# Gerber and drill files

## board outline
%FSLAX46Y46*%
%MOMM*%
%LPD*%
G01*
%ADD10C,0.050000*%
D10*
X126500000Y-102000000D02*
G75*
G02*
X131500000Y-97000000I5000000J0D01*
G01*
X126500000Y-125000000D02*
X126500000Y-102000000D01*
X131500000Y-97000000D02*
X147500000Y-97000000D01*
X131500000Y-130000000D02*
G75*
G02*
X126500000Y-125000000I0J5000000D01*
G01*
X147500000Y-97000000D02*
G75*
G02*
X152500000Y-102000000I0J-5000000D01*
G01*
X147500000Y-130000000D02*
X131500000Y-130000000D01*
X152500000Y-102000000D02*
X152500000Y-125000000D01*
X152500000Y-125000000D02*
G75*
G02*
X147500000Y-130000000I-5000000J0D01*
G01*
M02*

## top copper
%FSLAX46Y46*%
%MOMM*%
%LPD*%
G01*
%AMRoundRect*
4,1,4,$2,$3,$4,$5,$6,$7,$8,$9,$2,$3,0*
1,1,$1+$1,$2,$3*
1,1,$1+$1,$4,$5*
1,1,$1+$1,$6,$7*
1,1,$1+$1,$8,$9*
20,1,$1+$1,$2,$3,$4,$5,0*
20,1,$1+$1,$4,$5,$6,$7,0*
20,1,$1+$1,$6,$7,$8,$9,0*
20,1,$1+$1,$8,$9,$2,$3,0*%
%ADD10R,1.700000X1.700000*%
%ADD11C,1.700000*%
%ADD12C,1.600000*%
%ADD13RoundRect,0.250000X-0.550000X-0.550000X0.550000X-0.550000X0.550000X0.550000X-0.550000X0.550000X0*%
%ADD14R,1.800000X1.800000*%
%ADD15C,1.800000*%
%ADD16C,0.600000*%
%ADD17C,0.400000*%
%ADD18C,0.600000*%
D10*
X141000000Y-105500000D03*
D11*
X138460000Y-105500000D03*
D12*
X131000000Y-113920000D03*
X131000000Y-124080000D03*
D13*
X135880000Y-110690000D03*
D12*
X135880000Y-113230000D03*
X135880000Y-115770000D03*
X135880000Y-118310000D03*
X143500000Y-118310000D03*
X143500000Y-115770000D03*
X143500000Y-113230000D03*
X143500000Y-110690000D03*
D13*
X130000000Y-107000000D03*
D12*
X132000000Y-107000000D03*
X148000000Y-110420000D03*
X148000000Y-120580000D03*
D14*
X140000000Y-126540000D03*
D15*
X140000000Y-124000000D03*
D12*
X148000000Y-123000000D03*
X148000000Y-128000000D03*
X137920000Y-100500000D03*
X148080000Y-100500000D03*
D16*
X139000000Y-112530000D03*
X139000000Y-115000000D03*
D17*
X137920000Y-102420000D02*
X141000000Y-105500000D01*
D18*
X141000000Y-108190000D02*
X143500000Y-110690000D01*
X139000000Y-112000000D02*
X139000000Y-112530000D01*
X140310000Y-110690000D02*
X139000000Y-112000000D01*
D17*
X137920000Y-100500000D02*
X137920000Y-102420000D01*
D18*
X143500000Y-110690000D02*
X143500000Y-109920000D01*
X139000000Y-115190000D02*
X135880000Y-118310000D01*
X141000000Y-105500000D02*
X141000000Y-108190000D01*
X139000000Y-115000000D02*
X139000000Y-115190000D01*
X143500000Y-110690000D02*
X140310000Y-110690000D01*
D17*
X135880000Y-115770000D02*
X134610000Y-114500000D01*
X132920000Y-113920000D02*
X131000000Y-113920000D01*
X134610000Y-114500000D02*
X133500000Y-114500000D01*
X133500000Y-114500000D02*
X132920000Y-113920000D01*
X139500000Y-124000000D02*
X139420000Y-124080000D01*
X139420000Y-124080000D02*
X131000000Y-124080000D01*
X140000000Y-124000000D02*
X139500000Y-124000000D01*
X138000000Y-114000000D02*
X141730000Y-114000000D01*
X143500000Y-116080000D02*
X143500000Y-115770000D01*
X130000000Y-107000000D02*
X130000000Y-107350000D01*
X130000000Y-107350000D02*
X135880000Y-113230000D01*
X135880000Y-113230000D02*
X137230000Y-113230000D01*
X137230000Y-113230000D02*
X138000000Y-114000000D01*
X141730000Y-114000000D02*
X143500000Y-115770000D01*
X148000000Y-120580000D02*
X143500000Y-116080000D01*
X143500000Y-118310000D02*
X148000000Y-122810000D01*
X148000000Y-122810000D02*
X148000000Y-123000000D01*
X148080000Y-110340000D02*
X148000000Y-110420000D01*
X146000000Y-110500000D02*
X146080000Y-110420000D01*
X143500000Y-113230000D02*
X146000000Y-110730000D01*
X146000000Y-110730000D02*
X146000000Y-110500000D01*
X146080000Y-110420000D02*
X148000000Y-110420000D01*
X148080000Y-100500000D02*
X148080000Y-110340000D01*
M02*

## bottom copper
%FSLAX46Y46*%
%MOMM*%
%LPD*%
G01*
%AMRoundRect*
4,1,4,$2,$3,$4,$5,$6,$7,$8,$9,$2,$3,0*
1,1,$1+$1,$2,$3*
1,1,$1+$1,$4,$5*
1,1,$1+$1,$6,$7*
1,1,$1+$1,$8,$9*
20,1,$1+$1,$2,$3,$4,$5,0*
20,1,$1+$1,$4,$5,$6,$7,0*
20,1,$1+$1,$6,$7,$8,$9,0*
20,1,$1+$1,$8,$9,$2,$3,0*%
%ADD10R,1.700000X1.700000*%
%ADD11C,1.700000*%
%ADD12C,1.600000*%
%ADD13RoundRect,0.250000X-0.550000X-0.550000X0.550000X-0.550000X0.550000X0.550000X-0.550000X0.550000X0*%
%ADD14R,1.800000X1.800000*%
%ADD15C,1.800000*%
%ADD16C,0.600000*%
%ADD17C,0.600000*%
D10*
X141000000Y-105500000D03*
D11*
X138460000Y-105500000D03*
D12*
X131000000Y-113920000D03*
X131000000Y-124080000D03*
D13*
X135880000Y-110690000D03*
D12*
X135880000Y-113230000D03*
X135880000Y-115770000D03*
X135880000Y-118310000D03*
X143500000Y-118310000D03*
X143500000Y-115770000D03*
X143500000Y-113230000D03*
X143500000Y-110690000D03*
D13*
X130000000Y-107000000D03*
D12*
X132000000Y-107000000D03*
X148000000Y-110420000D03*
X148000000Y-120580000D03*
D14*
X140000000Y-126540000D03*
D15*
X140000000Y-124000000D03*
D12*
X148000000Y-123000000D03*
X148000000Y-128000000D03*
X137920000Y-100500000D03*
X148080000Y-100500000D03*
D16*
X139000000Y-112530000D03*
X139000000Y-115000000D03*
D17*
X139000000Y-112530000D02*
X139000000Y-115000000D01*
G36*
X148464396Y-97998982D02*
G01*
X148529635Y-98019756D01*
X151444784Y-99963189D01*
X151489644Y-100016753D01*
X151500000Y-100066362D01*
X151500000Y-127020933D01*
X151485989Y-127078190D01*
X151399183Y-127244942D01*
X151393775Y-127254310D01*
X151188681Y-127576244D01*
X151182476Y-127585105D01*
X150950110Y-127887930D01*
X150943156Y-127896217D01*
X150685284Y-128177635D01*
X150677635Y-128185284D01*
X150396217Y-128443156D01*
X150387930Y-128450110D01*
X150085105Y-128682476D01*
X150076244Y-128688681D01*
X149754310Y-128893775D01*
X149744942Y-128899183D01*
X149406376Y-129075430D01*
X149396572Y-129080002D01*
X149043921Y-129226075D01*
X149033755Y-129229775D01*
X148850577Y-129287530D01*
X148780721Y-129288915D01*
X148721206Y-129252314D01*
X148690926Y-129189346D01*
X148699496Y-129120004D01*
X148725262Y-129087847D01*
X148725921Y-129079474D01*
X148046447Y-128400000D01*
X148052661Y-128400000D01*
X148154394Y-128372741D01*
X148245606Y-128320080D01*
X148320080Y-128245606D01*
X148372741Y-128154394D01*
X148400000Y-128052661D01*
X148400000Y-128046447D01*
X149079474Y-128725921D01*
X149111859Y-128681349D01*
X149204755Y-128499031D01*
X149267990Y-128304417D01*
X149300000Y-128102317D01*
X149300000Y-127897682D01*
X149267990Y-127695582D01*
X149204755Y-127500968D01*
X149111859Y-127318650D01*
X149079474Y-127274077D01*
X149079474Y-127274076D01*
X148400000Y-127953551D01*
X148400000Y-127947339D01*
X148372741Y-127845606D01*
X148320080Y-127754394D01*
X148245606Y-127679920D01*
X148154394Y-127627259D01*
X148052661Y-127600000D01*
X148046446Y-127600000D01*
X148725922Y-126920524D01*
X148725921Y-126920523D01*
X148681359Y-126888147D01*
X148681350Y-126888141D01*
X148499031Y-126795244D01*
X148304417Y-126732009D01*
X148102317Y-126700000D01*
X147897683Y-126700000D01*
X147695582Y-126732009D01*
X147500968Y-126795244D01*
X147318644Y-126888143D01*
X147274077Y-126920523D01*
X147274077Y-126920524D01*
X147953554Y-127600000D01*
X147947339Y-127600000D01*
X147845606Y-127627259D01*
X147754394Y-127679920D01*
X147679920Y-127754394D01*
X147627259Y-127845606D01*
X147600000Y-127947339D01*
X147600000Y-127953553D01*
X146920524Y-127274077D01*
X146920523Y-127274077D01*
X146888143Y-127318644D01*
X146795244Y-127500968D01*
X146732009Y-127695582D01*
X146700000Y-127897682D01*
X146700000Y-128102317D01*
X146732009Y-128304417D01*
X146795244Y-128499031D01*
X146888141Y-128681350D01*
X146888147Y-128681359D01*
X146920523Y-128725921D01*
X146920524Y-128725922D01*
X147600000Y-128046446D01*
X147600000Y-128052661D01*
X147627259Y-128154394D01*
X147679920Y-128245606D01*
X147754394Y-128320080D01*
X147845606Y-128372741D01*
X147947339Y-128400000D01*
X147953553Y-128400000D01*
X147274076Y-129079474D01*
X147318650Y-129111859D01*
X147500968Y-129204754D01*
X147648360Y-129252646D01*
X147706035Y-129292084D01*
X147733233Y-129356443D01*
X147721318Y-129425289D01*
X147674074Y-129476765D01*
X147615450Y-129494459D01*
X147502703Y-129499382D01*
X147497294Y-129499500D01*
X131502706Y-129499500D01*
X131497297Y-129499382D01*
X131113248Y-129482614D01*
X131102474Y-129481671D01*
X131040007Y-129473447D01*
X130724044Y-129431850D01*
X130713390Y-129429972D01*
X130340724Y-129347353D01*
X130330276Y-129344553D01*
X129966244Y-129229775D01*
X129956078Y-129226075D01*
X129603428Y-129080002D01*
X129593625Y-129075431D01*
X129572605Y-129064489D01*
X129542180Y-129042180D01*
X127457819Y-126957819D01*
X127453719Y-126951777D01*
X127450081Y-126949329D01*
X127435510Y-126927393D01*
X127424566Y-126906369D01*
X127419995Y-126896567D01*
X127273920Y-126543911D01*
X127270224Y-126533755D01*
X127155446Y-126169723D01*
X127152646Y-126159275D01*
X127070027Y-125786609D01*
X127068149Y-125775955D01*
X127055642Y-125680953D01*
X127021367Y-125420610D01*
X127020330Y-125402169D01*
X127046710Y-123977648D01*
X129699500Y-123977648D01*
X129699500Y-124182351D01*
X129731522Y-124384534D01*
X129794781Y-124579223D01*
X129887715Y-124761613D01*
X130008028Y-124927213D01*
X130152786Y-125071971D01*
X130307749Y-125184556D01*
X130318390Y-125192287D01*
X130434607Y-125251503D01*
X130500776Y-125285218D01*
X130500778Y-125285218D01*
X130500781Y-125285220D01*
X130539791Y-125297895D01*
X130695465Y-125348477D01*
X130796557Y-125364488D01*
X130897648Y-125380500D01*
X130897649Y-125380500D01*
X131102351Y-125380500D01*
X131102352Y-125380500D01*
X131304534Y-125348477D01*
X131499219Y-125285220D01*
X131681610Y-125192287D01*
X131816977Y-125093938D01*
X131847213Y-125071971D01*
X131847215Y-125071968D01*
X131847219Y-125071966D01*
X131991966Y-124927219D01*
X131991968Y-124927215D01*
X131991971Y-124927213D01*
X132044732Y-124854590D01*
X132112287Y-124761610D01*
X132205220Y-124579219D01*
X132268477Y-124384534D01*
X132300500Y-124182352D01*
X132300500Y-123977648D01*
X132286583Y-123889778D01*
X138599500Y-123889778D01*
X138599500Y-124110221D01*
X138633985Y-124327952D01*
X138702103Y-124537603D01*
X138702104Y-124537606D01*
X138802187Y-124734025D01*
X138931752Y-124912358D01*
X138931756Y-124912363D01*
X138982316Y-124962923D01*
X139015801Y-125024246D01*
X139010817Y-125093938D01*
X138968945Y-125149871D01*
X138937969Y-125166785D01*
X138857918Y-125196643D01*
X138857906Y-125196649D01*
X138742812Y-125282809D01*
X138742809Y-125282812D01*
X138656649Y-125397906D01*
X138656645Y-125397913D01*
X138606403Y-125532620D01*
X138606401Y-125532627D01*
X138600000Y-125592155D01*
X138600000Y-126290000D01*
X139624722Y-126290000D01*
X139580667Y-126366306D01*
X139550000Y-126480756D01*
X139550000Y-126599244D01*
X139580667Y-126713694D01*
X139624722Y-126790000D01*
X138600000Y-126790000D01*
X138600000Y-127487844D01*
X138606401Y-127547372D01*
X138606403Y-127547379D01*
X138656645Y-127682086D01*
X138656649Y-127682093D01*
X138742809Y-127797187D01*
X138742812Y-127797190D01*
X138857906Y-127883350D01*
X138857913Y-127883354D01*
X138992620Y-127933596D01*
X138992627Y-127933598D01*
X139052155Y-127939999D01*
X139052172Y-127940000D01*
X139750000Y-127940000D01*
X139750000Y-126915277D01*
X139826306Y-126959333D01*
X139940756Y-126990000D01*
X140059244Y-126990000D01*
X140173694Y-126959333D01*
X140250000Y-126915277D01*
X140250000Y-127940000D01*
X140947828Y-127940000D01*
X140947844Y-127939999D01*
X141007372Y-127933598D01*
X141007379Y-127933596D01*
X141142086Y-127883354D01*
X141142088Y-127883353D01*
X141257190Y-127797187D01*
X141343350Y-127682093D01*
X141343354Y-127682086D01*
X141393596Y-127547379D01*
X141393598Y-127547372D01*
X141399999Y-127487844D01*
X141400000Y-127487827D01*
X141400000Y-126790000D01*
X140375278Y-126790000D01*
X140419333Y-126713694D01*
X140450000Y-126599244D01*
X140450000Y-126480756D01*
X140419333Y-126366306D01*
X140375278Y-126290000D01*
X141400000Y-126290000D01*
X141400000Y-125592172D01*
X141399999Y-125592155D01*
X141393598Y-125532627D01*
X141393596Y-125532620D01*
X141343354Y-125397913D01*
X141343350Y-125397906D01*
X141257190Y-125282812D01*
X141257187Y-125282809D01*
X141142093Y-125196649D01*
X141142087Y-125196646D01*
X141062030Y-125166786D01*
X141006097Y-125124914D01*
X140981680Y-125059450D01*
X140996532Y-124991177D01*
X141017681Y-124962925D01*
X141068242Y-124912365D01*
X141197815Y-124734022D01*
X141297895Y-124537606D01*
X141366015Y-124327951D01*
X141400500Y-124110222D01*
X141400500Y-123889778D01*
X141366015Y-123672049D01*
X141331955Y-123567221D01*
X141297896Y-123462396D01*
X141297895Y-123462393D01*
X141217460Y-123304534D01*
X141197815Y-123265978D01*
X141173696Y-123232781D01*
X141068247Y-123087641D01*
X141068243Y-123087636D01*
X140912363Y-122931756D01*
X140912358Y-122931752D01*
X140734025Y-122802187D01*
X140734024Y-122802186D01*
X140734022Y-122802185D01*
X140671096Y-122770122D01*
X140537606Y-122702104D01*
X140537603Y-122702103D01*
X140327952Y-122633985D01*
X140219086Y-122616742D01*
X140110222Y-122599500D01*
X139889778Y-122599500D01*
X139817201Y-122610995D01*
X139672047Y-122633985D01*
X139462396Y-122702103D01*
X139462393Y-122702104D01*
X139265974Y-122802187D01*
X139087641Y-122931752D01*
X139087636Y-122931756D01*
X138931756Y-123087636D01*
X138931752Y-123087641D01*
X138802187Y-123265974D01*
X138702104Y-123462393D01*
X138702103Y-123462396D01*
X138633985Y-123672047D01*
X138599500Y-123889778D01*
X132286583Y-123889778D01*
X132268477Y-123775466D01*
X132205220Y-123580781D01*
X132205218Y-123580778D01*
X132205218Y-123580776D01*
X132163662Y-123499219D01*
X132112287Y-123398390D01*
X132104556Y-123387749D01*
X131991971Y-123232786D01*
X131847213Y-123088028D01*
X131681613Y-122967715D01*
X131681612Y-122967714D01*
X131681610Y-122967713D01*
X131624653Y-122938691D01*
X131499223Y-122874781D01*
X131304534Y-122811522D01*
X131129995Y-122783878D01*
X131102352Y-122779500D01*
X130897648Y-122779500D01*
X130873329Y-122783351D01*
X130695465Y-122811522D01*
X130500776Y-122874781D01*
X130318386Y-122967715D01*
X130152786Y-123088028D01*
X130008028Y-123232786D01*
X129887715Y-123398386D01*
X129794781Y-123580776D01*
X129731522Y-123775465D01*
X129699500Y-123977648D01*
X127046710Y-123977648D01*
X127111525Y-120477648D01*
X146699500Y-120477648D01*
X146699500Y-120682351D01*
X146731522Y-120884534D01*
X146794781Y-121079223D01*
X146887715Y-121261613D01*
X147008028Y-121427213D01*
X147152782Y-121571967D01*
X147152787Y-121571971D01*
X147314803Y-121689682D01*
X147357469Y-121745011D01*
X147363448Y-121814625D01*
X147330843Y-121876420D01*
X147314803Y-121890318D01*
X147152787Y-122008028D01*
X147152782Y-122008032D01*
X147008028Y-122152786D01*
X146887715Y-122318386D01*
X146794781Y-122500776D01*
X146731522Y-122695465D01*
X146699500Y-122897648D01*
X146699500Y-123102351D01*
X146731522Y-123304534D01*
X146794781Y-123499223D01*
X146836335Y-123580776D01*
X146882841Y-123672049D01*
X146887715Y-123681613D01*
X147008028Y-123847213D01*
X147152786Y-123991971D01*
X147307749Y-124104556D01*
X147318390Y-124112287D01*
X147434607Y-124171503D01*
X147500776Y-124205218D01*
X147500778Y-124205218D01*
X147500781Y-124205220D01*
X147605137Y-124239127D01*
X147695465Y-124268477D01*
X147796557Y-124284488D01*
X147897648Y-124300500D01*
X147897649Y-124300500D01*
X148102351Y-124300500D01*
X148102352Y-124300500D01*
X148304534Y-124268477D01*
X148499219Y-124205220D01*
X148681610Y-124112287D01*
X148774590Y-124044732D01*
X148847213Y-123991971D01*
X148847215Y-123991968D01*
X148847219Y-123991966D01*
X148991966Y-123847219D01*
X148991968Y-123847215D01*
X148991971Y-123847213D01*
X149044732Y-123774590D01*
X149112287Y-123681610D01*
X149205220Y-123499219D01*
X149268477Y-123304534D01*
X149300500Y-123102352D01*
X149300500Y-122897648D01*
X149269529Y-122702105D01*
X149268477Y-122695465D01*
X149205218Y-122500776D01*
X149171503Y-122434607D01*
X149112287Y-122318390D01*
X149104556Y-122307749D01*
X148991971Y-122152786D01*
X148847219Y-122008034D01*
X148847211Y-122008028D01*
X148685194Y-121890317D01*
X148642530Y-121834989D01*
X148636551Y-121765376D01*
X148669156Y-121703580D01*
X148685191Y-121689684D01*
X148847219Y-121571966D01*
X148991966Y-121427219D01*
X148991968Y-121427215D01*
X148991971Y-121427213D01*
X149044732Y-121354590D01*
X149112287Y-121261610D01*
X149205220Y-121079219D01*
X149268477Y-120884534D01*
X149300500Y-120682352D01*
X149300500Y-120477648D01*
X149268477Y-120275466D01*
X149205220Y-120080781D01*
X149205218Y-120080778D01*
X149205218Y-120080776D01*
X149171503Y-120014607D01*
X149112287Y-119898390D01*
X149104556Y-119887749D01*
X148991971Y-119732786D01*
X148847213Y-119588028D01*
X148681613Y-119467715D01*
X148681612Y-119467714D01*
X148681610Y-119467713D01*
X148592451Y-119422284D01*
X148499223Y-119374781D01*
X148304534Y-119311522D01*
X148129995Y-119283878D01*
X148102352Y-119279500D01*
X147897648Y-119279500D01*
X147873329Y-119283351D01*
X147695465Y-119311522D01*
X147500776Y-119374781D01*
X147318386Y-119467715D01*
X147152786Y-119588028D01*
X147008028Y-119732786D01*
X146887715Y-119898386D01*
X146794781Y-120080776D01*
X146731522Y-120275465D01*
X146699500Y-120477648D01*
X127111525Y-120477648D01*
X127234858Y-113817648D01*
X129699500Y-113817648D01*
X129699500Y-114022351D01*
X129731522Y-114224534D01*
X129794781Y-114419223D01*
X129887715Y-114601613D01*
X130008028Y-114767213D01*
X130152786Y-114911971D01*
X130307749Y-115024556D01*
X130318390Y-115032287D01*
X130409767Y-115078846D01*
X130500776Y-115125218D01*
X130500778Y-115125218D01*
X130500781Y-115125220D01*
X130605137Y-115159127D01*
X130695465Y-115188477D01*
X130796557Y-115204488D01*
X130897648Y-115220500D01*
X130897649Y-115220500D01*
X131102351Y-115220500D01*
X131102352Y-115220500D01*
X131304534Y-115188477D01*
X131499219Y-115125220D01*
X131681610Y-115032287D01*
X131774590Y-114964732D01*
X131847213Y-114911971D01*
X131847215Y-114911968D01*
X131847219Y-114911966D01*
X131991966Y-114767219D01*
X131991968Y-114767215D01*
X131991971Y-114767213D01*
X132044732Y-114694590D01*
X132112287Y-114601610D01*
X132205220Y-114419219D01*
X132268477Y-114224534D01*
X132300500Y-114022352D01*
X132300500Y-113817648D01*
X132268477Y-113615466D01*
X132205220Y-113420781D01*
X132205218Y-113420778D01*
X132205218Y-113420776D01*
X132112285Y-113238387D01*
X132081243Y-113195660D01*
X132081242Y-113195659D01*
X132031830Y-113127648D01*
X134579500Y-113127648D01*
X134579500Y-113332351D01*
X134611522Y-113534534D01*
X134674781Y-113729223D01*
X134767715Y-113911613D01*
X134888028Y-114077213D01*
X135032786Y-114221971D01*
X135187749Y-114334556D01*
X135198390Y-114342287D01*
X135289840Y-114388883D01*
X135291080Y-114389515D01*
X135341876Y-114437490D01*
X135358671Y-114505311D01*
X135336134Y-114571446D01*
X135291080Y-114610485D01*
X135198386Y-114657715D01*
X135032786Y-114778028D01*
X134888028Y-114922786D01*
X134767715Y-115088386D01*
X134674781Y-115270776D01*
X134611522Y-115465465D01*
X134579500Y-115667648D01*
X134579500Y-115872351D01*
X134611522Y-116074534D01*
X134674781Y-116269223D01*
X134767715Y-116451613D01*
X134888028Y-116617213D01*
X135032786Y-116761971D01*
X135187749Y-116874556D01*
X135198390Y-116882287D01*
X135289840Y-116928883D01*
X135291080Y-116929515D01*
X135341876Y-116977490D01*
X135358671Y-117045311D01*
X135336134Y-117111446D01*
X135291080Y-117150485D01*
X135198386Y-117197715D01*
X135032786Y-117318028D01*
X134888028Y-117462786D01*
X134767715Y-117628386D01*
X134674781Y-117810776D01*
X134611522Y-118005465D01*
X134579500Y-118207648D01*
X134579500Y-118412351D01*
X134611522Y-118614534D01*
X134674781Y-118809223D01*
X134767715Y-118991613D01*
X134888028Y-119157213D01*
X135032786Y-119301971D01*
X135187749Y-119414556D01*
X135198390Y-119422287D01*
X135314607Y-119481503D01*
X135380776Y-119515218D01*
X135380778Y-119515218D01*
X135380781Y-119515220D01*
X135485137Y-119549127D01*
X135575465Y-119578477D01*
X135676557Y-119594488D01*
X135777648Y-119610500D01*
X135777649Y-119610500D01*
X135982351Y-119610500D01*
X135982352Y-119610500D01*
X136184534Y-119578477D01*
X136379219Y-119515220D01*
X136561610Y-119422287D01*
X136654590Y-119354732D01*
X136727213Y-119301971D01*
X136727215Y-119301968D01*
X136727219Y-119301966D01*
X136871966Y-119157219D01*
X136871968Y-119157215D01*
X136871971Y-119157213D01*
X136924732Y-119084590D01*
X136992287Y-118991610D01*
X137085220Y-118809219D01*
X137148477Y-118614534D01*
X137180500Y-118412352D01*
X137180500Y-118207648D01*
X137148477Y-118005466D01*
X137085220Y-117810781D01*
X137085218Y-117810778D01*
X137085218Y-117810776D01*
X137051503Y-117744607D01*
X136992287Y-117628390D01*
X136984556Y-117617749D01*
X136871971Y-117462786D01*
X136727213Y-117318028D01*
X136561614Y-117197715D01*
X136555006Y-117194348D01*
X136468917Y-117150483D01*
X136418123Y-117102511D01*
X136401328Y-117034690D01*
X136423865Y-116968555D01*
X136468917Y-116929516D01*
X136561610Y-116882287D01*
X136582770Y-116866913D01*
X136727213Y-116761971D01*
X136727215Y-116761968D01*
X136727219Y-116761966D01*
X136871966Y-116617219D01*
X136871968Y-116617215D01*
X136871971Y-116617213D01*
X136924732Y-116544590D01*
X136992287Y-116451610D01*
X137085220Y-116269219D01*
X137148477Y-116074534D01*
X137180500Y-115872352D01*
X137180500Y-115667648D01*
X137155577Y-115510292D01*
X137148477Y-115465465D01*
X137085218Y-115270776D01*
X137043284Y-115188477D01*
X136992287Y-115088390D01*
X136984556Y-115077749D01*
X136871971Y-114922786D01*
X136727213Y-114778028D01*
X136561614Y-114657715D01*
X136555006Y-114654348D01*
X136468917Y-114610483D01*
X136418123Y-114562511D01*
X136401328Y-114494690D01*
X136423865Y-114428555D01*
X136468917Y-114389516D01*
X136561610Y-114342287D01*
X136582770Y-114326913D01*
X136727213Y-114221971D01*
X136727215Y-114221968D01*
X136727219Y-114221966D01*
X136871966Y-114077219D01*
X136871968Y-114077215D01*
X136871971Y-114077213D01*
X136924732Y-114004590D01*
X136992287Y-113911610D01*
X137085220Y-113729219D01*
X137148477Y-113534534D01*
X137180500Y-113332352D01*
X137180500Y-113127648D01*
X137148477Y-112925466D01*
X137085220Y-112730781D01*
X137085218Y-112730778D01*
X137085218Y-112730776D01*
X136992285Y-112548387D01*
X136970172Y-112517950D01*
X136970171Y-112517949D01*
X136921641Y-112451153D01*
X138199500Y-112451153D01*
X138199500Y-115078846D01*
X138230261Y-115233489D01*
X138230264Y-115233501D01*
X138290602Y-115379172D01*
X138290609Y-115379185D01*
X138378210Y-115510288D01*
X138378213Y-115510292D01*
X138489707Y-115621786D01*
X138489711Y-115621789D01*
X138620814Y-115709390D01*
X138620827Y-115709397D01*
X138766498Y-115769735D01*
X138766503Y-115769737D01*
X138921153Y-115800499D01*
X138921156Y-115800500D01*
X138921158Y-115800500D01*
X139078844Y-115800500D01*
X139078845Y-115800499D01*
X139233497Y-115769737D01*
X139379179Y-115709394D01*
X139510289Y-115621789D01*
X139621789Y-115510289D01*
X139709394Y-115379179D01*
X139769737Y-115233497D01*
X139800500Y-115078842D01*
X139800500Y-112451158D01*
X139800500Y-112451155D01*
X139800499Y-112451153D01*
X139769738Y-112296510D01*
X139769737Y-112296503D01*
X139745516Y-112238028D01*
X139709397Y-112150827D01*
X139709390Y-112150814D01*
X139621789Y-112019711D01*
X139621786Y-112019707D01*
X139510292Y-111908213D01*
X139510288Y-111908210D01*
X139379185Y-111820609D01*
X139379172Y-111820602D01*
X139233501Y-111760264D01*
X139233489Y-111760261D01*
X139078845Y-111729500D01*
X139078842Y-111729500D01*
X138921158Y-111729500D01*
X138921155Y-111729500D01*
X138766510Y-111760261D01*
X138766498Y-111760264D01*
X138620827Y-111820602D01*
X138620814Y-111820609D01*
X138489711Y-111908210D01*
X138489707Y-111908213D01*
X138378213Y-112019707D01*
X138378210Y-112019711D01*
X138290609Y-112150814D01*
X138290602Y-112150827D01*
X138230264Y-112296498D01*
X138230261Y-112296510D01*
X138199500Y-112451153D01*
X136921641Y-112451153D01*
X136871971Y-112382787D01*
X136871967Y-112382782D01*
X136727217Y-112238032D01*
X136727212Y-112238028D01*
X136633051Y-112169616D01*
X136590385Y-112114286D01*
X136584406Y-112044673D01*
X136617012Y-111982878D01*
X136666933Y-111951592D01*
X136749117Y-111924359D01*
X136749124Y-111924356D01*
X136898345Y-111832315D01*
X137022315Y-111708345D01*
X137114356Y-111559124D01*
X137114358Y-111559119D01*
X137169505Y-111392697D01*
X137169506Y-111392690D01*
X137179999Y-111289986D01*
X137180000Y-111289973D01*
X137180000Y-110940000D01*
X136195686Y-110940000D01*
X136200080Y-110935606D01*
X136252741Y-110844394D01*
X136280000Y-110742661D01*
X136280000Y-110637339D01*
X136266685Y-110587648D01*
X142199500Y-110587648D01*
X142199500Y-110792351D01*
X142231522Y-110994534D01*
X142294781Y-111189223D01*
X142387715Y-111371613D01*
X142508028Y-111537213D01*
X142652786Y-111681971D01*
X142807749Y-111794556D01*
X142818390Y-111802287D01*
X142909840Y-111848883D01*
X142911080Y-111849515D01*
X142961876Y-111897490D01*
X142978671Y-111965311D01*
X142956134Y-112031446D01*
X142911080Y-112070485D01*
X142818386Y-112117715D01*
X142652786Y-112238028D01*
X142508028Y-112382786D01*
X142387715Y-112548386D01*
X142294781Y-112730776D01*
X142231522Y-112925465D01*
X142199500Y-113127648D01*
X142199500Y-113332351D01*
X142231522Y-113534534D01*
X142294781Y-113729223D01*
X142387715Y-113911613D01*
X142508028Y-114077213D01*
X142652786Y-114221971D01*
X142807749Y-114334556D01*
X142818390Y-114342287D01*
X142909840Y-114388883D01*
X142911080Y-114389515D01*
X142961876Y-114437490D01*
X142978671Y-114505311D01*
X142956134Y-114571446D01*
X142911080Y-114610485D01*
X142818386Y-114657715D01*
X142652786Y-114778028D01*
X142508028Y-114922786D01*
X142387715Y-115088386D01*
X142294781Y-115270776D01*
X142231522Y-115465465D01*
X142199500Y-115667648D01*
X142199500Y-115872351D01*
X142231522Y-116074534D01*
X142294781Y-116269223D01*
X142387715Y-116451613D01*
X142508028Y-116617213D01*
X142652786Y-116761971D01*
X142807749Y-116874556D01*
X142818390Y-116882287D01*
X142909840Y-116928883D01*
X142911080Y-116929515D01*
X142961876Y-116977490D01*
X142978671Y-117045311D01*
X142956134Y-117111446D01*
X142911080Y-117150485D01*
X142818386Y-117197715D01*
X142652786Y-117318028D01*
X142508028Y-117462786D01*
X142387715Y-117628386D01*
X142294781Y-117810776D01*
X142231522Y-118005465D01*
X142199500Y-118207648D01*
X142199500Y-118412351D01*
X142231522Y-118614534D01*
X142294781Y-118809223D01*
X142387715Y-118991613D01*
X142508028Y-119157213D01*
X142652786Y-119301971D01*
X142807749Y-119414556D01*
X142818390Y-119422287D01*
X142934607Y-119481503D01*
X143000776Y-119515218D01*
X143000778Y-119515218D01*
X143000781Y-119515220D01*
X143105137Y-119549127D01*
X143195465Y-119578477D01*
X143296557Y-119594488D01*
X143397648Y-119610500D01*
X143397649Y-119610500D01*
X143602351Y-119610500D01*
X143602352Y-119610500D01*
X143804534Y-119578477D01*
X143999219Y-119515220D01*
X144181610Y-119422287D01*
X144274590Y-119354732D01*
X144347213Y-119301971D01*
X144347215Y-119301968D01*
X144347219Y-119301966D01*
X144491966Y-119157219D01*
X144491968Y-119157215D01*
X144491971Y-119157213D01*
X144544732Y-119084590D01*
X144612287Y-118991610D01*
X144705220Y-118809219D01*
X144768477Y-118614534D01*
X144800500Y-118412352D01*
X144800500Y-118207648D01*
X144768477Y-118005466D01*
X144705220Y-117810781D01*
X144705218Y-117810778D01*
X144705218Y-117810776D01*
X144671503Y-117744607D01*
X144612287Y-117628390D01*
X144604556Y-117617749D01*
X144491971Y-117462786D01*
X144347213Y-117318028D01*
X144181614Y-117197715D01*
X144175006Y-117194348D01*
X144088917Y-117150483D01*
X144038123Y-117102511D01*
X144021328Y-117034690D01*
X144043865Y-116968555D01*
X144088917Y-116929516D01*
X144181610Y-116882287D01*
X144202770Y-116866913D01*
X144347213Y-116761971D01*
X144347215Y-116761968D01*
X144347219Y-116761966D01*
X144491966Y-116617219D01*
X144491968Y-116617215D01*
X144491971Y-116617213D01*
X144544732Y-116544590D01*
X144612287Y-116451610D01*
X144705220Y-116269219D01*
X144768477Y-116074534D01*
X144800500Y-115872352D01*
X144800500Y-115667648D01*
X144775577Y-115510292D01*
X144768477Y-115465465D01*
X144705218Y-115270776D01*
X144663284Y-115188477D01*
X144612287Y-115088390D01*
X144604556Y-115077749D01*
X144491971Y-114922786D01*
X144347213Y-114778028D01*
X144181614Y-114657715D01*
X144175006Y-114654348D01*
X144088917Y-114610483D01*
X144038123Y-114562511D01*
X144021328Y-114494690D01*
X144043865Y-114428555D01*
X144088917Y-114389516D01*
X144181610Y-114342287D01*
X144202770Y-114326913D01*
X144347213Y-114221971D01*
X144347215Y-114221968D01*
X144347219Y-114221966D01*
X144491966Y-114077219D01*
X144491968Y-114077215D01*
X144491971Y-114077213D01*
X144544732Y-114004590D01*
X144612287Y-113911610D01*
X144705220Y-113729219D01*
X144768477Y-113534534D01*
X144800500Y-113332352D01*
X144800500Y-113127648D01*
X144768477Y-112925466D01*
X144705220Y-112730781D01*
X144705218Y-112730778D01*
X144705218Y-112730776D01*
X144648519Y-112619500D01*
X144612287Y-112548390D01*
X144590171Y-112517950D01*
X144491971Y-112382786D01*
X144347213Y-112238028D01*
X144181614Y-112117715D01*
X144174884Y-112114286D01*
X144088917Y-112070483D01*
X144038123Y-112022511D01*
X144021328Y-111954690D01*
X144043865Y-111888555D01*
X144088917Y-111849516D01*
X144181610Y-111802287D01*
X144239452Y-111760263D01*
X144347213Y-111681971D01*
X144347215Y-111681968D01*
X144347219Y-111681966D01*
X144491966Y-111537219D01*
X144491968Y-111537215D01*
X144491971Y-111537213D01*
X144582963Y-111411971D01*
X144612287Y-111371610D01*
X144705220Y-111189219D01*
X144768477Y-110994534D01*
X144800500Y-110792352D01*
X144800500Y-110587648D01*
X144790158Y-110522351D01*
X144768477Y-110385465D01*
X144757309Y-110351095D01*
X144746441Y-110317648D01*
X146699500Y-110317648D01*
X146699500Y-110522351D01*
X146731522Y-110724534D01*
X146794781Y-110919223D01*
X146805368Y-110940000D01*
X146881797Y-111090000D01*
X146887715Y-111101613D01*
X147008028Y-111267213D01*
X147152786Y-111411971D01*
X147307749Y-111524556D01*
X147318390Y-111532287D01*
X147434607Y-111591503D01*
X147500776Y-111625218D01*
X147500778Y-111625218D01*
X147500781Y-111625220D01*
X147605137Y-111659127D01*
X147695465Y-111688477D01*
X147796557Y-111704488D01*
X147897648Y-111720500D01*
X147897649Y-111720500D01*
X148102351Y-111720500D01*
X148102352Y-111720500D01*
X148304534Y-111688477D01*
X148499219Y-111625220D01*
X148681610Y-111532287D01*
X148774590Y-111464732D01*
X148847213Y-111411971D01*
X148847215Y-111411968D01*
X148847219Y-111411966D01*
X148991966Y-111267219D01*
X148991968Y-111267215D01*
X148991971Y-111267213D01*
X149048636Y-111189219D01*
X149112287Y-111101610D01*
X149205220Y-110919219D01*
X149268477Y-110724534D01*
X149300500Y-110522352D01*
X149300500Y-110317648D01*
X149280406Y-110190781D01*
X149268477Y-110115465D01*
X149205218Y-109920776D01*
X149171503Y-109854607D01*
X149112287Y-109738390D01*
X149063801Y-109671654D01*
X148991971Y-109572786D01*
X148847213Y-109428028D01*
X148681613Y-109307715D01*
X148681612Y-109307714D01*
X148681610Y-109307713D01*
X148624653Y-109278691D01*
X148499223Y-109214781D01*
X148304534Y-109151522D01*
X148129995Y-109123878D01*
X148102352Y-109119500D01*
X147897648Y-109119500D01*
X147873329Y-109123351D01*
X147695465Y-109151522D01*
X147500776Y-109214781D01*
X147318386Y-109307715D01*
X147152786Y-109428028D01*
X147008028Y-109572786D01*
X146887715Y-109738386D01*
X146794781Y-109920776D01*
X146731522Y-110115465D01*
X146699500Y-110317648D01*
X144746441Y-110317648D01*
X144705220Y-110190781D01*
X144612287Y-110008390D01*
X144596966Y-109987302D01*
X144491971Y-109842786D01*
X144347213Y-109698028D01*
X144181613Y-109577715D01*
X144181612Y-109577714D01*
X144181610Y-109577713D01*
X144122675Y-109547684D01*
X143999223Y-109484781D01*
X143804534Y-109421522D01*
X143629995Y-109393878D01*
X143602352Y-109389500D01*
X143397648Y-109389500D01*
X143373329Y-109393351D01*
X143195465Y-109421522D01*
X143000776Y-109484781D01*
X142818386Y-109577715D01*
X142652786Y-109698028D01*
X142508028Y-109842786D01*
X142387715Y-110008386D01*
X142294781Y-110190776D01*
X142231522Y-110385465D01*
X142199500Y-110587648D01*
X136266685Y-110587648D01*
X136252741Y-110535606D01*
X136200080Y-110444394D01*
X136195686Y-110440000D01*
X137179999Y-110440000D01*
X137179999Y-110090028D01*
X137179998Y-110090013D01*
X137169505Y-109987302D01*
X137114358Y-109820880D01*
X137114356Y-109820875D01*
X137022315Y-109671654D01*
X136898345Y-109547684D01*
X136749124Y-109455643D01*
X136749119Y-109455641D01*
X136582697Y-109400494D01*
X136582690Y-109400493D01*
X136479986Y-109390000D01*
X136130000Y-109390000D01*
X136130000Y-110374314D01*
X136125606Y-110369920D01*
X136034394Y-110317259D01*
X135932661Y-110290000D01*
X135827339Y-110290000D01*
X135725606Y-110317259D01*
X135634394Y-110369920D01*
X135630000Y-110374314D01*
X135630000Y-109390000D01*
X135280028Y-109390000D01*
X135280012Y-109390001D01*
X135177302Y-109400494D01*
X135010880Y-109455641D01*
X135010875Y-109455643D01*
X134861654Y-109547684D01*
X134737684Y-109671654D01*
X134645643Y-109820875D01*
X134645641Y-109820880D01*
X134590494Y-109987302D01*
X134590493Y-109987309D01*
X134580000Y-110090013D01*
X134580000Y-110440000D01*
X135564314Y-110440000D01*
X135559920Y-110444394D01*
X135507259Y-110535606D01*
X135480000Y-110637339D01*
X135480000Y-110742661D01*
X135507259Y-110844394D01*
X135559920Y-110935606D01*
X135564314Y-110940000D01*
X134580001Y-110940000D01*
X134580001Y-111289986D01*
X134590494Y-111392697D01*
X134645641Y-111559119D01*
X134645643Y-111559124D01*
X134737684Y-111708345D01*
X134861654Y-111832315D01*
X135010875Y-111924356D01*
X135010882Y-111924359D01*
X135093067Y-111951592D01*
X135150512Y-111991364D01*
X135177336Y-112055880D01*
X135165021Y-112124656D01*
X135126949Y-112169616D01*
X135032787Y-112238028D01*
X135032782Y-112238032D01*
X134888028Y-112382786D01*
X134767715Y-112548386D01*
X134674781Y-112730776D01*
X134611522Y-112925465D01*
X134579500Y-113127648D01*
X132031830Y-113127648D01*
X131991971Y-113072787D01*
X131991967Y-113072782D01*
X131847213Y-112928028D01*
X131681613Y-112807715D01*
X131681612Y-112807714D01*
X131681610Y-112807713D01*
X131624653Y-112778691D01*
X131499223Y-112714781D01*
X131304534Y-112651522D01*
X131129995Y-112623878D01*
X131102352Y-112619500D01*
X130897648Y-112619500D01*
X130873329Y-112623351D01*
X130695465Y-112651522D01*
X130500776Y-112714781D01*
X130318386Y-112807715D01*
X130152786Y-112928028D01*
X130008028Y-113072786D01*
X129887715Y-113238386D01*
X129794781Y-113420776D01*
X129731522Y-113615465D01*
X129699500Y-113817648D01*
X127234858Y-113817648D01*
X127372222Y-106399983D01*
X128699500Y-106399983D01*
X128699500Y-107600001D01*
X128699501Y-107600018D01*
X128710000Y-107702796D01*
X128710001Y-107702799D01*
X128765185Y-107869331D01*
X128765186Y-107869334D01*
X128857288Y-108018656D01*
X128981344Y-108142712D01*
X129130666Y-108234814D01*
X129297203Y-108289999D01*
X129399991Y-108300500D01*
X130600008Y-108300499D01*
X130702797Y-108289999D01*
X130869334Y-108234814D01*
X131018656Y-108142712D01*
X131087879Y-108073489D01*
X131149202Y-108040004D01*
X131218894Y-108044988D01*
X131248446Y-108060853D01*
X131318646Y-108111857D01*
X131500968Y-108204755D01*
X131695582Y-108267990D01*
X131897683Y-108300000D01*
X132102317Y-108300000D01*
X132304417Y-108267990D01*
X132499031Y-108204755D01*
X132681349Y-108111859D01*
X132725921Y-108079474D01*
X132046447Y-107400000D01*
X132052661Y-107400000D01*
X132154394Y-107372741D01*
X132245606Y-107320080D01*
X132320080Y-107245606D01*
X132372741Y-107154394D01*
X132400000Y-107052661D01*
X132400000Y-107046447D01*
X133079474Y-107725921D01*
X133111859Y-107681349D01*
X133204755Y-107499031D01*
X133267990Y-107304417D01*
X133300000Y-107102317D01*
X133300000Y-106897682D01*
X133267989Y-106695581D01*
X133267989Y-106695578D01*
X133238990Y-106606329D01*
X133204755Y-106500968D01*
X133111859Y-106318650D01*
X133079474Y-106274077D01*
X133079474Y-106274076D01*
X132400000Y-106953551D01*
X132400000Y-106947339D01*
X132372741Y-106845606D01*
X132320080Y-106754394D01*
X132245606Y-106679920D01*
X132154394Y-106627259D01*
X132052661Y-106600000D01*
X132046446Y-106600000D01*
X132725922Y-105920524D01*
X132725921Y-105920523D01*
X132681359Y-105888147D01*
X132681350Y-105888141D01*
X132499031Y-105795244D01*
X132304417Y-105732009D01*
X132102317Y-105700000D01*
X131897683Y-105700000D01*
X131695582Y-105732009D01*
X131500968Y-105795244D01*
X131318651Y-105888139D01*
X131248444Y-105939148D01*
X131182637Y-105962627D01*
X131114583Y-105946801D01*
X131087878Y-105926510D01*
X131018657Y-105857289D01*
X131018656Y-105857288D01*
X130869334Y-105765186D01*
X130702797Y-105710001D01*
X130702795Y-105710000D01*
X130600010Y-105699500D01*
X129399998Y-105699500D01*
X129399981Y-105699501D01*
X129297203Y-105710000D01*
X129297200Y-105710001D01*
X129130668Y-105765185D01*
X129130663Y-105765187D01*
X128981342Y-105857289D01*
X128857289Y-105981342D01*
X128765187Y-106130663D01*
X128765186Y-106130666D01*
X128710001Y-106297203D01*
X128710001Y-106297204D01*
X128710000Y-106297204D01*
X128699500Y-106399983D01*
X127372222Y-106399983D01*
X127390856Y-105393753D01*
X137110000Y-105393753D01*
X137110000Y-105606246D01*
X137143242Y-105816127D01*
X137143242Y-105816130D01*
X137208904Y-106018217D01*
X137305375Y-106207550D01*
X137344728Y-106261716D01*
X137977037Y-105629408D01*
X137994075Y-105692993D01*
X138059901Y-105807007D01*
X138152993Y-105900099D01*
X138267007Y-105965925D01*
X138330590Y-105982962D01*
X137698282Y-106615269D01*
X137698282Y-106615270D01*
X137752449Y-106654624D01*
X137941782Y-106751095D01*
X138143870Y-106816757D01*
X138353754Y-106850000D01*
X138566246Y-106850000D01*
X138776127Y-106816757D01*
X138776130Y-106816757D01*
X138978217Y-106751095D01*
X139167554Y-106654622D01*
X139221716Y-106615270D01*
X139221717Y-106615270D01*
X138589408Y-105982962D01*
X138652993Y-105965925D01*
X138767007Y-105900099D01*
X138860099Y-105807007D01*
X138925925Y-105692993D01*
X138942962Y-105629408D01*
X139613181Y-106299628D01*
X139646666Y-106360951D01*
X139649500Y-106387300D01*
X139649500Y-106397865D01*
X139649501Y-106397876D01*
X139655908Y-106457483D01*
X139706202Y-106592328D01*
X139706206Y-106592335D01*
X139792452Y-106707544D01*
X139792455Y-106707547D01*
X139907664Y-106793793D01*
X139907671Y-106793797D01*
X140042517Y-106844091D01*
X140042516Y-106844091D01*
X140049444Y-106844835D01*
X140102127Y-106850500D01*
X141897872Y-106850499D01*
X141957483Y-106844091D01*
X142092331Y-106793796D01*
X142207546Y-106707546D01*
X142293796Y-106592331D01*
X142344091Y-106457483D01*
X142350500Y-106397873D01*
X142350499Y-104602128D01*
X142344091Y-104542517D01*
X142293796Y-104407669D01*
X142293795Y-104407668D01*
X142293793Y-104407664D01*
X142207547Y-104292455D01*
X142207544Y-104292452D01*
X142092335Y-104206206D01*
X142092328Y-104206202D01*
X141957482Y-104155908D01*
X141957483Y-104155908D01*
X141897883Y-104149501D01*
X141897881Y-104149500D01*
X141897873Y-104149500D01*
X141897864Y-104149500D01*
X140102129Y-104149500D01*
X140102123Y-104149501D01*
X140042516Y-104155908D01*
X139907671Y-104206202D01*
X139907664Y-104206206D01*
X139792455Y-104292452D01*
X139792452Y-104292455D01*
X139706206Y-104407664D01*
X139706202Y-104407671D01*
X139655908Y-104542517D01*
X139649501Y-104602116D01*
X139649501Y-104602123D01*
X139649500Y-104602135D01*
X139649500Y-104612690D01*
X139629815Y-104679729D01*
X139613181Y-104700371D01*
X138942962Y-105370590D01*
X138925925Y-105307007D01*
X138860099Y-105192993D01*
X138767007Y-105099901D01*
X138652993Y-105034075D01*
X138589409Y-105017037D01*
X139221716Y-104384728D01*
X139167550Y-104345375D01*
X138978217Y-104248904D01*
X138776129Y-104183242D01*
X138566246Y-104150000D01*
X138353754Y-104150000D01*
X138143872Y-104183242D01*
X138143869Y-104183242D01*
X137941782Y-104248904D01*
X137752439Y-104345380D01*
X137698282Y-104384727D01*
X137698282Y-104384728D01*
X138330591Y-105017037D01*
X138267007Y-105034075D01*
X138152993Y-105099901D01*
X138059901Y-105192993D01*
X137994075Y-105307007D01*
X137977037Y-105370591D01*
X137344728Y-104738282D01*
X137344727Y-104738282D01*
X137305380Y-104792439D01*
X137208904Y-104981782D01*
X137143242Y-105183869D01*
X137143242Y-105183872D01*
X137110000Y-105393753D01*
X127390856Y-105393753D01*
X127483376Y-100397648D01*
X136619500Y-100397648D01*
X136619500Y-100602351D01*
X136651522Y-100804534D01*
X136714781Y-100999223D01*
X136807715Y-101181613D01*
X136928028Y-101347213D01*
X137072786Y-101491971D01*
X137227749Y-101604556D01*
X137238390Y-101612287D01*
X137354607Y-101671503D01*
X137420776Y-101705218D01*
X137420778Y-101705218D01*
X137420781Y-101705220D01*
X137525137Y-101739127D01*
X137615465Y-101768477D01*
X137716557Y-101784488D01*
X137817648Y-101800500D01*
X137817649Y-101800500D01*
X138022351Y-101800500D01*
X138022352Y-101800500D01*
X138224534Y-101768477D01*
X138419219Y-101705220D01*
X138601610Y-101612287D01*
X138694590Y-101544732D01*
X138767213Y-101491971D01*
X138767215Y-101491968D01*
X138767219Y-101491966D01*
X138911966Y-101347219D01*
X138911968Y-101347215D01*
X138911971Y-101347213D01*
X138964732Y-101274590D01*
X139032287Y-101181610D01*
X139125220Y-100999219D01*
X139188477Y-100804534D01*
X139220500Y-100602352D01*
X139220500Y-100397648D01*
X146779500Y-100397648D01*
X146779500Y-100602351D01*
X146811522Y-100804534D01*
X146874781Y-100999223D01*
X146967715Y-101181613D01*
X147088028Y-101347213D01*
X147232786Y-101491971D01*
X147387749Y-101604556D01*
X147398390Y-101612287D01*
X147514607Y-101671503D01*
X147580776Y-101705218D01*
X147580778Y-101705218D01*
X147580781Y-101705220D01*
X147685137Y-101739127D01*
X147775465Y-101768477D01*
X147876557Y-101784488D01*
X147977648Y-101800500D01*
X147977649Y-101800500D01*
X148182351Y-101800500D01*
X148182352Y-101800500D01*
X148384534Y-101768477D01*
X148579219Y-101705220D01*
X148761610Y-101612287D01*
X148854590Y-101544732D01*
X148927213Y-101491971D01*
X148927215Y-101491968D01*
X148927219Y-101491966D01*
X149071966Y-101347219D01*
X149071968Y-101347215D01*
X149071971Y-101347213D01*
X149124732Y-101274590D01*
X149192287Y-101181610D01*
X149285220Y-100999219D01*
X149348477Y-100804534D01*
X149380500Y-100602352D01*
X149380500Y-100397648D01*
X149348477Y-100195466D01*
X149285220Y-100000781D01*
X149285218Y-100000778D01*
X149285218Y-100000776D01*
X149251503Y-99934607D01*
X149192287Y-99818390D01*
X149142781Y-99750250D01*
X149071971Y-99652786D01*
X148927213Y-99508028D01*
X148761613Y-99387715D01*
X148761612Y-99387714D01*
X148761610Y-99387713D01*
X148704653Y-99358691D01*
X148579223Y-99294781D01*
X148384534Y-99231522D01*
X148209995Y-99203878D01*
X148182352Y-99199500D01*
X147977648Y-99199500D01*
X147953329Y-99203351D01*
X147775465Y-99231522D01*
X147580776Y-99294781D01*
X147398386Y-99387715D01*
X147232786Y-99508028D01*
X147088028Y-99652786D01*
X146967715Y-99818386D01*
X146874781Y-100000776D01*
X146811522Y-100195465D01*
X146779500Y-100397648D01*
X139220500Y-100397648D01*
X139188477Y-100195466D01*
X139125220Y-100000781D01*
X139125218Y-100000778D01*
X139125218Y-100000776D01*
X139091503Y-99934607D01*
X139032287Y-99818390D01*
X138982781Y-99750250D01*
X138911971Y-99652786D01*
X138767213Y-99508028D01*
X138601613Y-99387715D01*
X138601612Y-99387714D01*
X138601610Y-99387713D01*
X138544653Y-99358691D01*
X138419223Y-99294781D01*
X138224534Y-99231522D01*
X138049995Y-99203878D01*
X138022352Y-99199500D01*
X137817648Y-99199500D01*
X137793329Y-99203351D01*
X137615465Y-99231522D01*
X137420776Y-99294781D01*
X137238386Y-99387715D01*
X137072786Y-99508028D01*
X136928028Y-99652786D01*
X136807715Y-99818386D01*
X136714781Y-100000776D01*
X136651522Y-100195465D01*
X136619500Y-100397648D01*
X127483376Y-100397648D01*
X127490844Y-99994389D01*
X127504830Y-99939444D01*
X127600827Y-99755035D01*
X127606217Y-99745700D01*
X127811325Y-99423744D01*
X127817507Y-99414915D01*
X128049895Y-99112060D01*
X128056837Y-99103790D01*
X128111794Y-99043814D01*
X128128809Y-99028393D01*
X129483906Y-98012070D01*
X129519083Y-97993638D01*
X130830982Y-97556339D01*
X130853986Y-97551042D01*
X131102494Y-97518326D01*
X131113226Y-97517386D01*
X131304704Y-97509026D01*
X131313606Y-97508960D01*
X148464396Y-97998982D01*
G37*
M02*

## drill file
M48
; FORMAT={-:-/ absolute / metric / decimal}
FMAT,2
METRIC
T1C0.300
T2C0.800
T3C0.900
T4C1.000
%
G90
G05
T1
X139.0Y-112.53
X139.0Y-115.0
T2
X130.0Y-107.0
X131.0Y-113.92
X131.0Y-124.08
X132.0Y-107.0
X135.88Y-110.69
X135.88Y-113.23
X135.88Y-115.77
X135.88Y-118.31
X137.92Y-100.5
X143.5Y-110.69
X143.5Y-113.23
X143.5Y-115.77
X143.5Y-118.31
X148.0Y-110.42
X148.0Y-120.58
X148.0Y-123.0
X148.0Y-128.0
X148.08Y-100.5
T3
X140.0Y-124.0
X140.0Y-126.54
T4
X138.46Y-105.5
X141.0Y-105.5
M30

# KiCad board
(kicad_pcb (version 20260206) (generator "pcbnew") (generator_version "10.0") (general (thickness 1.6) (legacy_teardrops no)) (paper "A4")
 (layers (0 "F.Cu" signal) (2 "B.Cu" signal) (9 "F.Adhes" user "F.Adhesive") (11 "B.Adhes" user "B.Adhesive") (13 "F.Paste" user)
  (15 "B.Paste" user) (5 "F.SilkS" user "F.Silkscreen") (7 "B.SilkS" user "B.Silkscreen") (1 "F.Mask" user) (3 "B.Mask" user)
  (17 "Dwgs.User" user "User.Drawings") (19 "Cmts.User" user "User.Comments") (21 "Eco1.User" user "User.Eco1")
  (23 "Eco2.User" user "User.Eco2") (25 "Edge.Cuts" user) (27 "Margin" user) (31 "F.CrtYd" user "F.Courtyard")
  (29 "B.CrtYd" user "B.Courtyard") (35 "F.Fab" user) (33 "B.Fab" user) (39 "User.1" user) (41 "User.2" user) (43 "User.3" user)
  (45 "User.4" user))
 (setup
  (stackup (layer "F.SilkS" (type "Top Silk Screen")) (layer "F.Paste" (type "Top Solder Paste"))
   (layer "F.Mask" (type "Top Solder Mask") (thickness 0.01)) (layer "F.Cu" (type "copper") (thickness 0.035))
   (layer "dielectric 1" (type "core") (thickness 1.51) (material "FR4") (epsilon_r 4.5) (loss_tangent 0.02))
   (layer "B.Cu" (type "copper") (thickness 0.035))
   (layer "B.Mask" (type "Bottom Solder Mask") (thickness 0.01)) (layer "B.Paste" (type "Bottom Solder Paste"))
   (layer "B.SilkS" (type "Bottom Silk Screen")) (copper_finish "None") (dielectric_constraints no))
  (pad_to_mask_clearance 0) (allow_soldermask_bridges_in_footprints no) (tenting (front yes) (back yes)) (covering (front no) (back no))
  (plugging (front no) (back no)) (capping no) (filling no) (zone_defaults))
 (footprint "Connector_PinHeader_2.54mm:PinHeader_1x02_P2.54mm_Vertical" (layer "F.Cu") (at 141 105.5 -90)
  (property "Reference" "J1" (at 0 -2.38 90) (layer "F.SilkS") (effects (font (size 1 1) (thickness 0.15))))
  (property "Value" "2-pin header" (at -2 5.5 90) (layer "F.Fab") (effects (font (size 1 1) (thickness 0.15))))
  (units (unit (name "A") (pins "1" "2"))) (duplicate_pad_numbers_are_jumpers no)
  (pad "1" thru_hole rect (at 0 0 270) (size 1.7 1.7) (drill 1) (layers "*.Cu" "*.Mask") (remove_unused_layers no) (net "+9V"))
  (pad "2" thru_hole circle (at 0 2.54 270) (size 1.7 1.7) (drill 1) (layers "*.Cu" "*.Mask") (remove_unused_layers no) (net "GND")))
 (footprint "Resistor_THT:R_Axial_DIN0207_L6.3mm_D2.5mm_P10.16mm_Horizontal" (layer "F.Cu") (at 131 113.92 -90)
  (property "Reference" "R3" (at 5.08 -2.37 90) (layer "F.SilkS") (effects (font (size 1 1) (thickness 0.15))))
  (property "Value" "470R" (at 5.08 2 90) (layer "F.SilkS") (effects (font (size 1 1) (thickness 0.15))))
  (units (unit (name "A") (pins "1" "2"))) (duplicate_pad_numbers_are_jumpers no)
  (pad "1" thru_hole circle (at 0 0 270) (size 1.6 1.6) (drill 0.8) (layers "*.Cu" "*.Mask") (remove_unused_layers no) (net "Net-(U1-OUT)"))
  (pad "2" thru_hole circle (at 10.16 0 270) (size 1.6 1.6) (drill 0.8) (layers "*.Cu" "*.Mask") (remove_unused_layers no)
   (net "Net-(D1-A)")))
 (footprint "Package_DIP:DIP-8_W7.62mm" (layer "F.Cu") (at 135.88 110.69)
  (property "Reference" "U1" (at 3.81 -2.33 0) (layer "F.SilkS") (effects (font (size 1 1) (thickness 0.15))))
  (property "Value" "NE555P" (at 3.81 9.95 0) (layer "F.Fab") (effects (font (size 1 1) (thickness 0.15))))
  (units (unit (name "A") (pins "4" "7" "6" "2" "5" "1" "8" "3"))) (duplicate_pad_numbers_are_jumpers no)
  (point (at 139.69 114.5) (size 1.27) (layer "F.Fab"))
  (pad "1" thru_hole roundrect (at 0 0) (size 1.6 1.6) (drill 0.8) (layers "*.Cu" "*.Mask") (remove_unused_layers no)
   (roundrect_rratio 0.15625) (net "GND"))
  (pad "2" thru_hole circle (at 0 2.54) (size 1.6 1.6) (drill 0.8) (layers "*.Cu" "*.Mask") (remove_unused_layers no) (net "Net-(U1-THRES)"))
  (pad "3" thru_hole circle (at 0 5.08) (size 1.6 1.6) (drill 0.8) (layers "*.Cu" "*.Mask") (remove_unused_layers no) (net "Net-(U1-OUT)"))
  (pad "4" thru_hole circle (at 0 7.62) (size 1.6 1.6) (drill 0.8) (layers "*.Cu" "*.Mask") (remove_unused_layers no) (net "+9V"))
  (pad "5" thru_hole circle (at 7.62 7.62) (size 1.6 1.6) (drill 0.8) (layers "*.Cu" "*.Mask") (remove_unused_layers no)
   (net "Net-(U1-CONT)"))
  (pad "6" thru_hole circle (at 7.62 5.08) (size 1.6 1.6) (drill 0.8) (layers "*.Cu" "*.Mask") (remove_unused_layers no)
   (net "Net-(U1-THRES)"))
  (pad "7" thru_hole circle (at 7.62 2.54) (size 1.6 1.6) (drill 0.8) (layers "*.Cu" "*.Mask") (remove_unused_layers no)
   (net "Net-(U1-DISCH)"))
  (pad "8" thru_hole circle (at 7.62 0) (size 1.6 1.6) (drill 0.8) (layers "*.Cu" "*.Mask") (remove_unused_layers no) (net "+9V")))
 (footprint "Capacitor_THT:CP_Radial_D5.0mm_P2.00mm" (layer "F.Cu") (at 130 107)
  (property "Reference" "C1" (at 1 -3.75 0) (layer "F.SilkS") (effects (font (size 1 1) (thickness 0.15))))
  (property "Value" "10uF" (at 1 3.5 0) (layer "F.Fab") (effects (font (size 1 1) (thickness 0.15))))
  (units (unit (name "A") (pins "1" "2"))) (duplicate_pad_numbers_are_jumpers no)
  (pad "1" thru_hole roundrect (at 0 0) (size 1.6 1.6) (drill 0.8) (layers "*.Cu" "*.Mask") (remove_unused_layers no)
   (roundrect_rratio 0.15625) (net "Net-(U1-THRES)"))
  (pad "2" thru_hole circle (at 2 0) (size 1.6 1.6) (drill 0.8) (layers "*.Cu" "*.Mask") (remove_unused_layers no) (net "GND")))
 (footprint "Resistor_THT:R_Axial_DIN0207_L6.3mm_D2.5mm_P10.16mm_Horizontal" (layer "F.Cu") (at 148 110.42 -90)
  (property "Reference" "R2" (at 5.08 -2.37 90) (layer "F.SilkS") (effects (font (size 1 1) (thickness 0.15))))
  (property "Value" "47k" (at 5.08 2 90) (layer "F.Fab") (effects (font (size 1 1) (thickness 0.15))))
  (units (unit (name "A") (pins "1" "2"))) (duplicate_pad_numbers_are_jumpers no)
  (pad "1" thru_hole circle (at 0 0 270) (size 1.6 1.6) (drill 0.8) (layers "*.Cu" "*.Mask") (remove_unused_layers no)
   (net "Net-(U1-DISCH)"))
  (pad "2" thru_hole circle (at 10.16 0 270) (size 1.6 1.6) (drill 0.8) (layers "*.Cu" "*.Mask") (remove_unused_layers no)
   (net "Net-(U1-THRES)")))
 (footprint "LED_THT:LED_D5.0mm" (layer "F.Cu") (at 140 126.54 90)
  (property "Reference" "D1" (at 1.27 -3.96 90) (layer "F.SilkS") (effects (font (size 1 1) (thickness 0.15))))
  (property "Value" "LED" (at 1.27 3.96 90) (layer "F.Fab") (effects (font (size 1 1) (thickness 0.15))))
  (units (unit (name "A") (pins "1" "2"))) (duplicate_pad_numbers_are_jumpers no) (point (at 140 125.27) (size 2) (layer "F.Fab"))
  (pad "1" thru_hole rect (at 0 0 90) (size 1.8 1.8) (drill 0.9) (layers "*.Cu" "*.Mask") (remove_unused_layers no) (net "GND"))
  (pad "2" thru_hole circle (at 2.54 0 90) (size 1.8 1.8) (drill 0.9) (layers "*.Cu" "*.Mask") (remove_unused_layers no) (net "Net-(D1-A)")))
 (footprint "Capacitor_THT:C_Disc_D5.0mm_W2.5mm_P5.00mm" (layer "F.Cu") (at 148 123 -90)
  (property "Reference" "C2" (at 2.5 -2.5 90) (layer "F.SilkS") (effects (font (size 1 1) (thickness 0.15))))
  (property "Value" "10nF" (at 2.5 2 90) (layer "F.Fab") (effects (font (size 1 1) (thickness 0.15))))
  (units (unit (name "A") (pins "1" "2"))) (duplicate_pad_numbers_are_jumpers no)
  (pad "1" thru_hole circle (at 0 0 270) (size 1.6 1.6) (drill 0.8) (layers "*.Cu" "*.Mask") (remove_unused_layers no) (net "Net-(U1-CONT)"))
  (pad "2" thru_hole circle (at 5 0 270) (size 1.6 1.6) (drill 0.8) (layers "*.Cu" "*.Mask") (remove_unused_layers no) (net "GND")))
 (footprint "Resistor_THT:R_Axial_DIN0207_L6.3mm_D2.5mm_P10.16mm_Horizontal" (layer "F.Cu") (at 137.92 100.5)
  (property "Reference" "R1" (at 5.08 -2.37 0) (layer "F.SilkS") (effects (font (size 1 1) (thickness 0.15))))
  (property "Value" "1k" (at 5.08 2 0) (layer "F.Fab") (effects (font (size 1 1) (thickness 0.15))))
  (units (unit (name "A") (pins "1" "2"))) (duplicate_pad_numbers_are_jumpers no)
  (pad "1" thru_hole circle (at 0 0) (size 1.6 1.6) (drill 0.8) (layers "*.Cu" "*.Mask") (remove_unused_layers no) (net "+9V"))
  (pad "2" thru_hole circle (at 10.16 0) (size 1.6 1.6) (drill 0.8) (layers "*.Cu" "*.Mask") (remove_unused_layers no)
   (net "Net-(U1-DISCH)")))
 (gr_arc (start 126.5 102) (mid 127.964466 98.464466) (end 131.5 97) (stroke (width 0.05) (type default)) (layer "Edge.Cuts"))
 (gr_line (start 126.5 125) (end 126.5 102) (stroke (width 0.05) (type default)) (layer "Edge.Cuts"))
 (gr_line (start 131.5 97) (end 147.5 97) (stroke (width 0.05) (type default)) (layer "Edge.Cuts"))
 (gr_arc (start 131.5 130) (mid 127.964466 128.535534) (end 126.5 125) (stroke (width 0.05) (type default)) (layer "Edge.Cuts"))
 (gr_arc (start 147.5 97) (mid 151.035534 98.464466) (end 152.5 102) (stroke (width 0.05) (type default)) (layer "Edge.Cuts"))
 (gr_line (start 147.5 130) (end 131.5 130) (stroke (width 0.05) (type default)) (layer "Edge.Cuts"))
 (gr_line (start 152.5 102) (end 152.5 125) (stroke (width 0.05) (type default)) (layer "Edge.Cuts"))
 (gr_arc (start 152.5 125) (mid 151.035534 128.535534) (end 147.5 130) (stroke (width 0.05) (type default)) (layer "Edge.Cuts"))
 (segment (start 137.92 102.42) (end 141 105.5) (width 0.4) (layer "F.Cu") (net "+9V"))
 (segment (start 141 108.19) (end 143.5 110.69) (width 0.6) (layer "F.Cu") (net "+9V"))
 (segment (start 139 112) (end 139 112.53) (width 0.6) (layer "F.Cu") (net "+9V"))
 (segment (start 140.31 110.69) (end 139 112) (width 0.6) (layer "F.Cu") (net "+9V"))
 (segment (start 137.92 100.5) (end 137.92 102.42) (width 0.4) (layer "F.Cu") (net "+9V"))
 (segment (start 143.5 110.69) (end 143.5 109.92) (width 0.6) (layer "F.Cu") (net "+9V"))
 (segment (start 139 115.19) (end 135.88 118.31) (width 0.6) (layer "F.Cu") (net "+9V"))
 (segment (start 141 105.5) (end 141 108.19) (width 0.6) (layer "F.Cu") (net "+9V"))
 (segment (start 139 115) (end 139 115.19) (width 0.6) (layer "F.Cu") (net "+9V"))
 (segment (start 143.5 110.69) (end 140.31 110.69) (width 0.6) (layer "F.Cu") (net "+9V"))
 (via (at 139 112.53) (size 0.6) (drill 0.3) (layers "F.Cu" "B.Cu") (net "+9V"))
 (via (at 139 115) (size 0.6) (drill 0.3) (layers "F.Cu" "B.Cu") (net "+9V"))
 (segment (start 139 112.53) (end 139 115) (width 0.6) (layer "B.Cu") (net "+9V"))
 (segment (start 135.88 115.77) (end 134.61 114.5) (width 0.4) (layer "F.Cu") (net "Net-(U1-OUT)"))
 (segment (start 132.92 113.92) (end 131 113.92) (width 0.4) (layer "F.Cu") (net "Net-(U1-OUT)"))
 (segment (start 134.61 114.5) (end 133.5 114.5) (width 0.4) (layer "F.Cu") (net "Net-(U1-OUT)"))
 (segment (start 133.5 114.5) (end 132.92 113.92) (width 0.4) (layer "F.Cu") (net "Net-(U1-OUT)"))
 (segment (start 139.5 124) (end 139.42 124.08) (width 0.4) (layer "F.Cu") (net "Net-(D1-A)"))
 (segment (start 139.42 124.08) (end 131 124.08) (width 0.4) (layer "F.Cu") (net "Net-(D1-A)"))
 (segment (start 140 124) (end 139.5 124) (width 0.4) (layer "F.Cu") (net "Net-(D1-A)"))
 (segment (start 138 114) (end 141.73 114) (width 0.4) (layer "F.Cu") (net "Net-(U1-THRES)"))
 (segment (start 143.5 116.08) (end 143.5 115.77) (width 0.4) (layer "F.Cu") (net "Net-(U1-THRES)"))
 (segment (start 130 107) (end 130 107.35) (width 0.4) (layer "F.Cu") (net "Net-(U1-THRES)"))
 (segment (start 130 107.35) (end 135.88 113.23) (width 0.4) (layer "F.Cu") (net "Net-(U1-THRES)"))
 (segment (start 135.88 113.23) (end 137.23 113.23) (width 0.4) (layer "F.Cu") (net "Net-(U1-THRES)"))
 (segment (start 137.23 113.23) (end 138 114) (width 0.4) (layer "F.Cu") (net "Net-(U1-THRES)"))
 (segment (start 141.73 114) (end 143.5 115.77) (width 0.4) (layer "F.Cu") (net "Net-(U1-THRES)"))
 (segment (start 148 120.58) (end 143.5 116.08) (width 0.4) (layer "F.Cu") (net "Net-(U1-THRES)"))
 (segment (start 143.5 118.31) (end 148 122.81) (width 0.4) (layer "F.Cu") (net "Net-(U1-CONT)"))
 (segment (start 148 122.81) (end 148 123) (width 0.4) (layer "F.Cu") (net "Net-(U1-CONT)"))
 (segment (start 148.08 110.34) (end 148 110.42) (width 0.4) (layer "F.Cu") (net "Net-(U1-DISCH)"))
 (segment (start 146 110.5) (end 146.08 110.42) (width 0.4) (layer "F.Cu") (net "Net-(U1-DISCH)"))
 (segment (start 143.5 113.23) (end 146 110.73) (width 0.4) (layer "F.Cu") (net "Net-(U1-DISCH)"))
 (segment (start 146 110.73) (end 146 110.5) (width 0.4) (layer "F.Cu") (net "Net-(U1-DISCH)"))
 (segment (start 146.08 110.42) (end 148 110.42) (width 0.4) (layer "F.Cu") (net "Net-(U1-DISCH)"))
 (segment (start 148.08 100.5) (end 148.08 110.34) (width 0.4) (layer "F.Cu") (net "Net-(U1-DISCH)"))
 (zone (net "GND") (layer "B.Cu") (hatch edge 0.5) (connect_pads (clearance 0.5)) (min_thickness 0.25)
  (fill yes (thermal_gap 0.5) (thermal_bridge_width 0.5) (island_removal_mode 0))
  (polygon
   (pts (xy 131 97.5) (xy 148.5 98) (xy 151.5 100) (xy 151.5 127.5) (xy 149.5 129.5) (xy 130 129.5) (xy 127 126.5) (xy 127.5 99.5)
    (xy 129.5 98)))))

